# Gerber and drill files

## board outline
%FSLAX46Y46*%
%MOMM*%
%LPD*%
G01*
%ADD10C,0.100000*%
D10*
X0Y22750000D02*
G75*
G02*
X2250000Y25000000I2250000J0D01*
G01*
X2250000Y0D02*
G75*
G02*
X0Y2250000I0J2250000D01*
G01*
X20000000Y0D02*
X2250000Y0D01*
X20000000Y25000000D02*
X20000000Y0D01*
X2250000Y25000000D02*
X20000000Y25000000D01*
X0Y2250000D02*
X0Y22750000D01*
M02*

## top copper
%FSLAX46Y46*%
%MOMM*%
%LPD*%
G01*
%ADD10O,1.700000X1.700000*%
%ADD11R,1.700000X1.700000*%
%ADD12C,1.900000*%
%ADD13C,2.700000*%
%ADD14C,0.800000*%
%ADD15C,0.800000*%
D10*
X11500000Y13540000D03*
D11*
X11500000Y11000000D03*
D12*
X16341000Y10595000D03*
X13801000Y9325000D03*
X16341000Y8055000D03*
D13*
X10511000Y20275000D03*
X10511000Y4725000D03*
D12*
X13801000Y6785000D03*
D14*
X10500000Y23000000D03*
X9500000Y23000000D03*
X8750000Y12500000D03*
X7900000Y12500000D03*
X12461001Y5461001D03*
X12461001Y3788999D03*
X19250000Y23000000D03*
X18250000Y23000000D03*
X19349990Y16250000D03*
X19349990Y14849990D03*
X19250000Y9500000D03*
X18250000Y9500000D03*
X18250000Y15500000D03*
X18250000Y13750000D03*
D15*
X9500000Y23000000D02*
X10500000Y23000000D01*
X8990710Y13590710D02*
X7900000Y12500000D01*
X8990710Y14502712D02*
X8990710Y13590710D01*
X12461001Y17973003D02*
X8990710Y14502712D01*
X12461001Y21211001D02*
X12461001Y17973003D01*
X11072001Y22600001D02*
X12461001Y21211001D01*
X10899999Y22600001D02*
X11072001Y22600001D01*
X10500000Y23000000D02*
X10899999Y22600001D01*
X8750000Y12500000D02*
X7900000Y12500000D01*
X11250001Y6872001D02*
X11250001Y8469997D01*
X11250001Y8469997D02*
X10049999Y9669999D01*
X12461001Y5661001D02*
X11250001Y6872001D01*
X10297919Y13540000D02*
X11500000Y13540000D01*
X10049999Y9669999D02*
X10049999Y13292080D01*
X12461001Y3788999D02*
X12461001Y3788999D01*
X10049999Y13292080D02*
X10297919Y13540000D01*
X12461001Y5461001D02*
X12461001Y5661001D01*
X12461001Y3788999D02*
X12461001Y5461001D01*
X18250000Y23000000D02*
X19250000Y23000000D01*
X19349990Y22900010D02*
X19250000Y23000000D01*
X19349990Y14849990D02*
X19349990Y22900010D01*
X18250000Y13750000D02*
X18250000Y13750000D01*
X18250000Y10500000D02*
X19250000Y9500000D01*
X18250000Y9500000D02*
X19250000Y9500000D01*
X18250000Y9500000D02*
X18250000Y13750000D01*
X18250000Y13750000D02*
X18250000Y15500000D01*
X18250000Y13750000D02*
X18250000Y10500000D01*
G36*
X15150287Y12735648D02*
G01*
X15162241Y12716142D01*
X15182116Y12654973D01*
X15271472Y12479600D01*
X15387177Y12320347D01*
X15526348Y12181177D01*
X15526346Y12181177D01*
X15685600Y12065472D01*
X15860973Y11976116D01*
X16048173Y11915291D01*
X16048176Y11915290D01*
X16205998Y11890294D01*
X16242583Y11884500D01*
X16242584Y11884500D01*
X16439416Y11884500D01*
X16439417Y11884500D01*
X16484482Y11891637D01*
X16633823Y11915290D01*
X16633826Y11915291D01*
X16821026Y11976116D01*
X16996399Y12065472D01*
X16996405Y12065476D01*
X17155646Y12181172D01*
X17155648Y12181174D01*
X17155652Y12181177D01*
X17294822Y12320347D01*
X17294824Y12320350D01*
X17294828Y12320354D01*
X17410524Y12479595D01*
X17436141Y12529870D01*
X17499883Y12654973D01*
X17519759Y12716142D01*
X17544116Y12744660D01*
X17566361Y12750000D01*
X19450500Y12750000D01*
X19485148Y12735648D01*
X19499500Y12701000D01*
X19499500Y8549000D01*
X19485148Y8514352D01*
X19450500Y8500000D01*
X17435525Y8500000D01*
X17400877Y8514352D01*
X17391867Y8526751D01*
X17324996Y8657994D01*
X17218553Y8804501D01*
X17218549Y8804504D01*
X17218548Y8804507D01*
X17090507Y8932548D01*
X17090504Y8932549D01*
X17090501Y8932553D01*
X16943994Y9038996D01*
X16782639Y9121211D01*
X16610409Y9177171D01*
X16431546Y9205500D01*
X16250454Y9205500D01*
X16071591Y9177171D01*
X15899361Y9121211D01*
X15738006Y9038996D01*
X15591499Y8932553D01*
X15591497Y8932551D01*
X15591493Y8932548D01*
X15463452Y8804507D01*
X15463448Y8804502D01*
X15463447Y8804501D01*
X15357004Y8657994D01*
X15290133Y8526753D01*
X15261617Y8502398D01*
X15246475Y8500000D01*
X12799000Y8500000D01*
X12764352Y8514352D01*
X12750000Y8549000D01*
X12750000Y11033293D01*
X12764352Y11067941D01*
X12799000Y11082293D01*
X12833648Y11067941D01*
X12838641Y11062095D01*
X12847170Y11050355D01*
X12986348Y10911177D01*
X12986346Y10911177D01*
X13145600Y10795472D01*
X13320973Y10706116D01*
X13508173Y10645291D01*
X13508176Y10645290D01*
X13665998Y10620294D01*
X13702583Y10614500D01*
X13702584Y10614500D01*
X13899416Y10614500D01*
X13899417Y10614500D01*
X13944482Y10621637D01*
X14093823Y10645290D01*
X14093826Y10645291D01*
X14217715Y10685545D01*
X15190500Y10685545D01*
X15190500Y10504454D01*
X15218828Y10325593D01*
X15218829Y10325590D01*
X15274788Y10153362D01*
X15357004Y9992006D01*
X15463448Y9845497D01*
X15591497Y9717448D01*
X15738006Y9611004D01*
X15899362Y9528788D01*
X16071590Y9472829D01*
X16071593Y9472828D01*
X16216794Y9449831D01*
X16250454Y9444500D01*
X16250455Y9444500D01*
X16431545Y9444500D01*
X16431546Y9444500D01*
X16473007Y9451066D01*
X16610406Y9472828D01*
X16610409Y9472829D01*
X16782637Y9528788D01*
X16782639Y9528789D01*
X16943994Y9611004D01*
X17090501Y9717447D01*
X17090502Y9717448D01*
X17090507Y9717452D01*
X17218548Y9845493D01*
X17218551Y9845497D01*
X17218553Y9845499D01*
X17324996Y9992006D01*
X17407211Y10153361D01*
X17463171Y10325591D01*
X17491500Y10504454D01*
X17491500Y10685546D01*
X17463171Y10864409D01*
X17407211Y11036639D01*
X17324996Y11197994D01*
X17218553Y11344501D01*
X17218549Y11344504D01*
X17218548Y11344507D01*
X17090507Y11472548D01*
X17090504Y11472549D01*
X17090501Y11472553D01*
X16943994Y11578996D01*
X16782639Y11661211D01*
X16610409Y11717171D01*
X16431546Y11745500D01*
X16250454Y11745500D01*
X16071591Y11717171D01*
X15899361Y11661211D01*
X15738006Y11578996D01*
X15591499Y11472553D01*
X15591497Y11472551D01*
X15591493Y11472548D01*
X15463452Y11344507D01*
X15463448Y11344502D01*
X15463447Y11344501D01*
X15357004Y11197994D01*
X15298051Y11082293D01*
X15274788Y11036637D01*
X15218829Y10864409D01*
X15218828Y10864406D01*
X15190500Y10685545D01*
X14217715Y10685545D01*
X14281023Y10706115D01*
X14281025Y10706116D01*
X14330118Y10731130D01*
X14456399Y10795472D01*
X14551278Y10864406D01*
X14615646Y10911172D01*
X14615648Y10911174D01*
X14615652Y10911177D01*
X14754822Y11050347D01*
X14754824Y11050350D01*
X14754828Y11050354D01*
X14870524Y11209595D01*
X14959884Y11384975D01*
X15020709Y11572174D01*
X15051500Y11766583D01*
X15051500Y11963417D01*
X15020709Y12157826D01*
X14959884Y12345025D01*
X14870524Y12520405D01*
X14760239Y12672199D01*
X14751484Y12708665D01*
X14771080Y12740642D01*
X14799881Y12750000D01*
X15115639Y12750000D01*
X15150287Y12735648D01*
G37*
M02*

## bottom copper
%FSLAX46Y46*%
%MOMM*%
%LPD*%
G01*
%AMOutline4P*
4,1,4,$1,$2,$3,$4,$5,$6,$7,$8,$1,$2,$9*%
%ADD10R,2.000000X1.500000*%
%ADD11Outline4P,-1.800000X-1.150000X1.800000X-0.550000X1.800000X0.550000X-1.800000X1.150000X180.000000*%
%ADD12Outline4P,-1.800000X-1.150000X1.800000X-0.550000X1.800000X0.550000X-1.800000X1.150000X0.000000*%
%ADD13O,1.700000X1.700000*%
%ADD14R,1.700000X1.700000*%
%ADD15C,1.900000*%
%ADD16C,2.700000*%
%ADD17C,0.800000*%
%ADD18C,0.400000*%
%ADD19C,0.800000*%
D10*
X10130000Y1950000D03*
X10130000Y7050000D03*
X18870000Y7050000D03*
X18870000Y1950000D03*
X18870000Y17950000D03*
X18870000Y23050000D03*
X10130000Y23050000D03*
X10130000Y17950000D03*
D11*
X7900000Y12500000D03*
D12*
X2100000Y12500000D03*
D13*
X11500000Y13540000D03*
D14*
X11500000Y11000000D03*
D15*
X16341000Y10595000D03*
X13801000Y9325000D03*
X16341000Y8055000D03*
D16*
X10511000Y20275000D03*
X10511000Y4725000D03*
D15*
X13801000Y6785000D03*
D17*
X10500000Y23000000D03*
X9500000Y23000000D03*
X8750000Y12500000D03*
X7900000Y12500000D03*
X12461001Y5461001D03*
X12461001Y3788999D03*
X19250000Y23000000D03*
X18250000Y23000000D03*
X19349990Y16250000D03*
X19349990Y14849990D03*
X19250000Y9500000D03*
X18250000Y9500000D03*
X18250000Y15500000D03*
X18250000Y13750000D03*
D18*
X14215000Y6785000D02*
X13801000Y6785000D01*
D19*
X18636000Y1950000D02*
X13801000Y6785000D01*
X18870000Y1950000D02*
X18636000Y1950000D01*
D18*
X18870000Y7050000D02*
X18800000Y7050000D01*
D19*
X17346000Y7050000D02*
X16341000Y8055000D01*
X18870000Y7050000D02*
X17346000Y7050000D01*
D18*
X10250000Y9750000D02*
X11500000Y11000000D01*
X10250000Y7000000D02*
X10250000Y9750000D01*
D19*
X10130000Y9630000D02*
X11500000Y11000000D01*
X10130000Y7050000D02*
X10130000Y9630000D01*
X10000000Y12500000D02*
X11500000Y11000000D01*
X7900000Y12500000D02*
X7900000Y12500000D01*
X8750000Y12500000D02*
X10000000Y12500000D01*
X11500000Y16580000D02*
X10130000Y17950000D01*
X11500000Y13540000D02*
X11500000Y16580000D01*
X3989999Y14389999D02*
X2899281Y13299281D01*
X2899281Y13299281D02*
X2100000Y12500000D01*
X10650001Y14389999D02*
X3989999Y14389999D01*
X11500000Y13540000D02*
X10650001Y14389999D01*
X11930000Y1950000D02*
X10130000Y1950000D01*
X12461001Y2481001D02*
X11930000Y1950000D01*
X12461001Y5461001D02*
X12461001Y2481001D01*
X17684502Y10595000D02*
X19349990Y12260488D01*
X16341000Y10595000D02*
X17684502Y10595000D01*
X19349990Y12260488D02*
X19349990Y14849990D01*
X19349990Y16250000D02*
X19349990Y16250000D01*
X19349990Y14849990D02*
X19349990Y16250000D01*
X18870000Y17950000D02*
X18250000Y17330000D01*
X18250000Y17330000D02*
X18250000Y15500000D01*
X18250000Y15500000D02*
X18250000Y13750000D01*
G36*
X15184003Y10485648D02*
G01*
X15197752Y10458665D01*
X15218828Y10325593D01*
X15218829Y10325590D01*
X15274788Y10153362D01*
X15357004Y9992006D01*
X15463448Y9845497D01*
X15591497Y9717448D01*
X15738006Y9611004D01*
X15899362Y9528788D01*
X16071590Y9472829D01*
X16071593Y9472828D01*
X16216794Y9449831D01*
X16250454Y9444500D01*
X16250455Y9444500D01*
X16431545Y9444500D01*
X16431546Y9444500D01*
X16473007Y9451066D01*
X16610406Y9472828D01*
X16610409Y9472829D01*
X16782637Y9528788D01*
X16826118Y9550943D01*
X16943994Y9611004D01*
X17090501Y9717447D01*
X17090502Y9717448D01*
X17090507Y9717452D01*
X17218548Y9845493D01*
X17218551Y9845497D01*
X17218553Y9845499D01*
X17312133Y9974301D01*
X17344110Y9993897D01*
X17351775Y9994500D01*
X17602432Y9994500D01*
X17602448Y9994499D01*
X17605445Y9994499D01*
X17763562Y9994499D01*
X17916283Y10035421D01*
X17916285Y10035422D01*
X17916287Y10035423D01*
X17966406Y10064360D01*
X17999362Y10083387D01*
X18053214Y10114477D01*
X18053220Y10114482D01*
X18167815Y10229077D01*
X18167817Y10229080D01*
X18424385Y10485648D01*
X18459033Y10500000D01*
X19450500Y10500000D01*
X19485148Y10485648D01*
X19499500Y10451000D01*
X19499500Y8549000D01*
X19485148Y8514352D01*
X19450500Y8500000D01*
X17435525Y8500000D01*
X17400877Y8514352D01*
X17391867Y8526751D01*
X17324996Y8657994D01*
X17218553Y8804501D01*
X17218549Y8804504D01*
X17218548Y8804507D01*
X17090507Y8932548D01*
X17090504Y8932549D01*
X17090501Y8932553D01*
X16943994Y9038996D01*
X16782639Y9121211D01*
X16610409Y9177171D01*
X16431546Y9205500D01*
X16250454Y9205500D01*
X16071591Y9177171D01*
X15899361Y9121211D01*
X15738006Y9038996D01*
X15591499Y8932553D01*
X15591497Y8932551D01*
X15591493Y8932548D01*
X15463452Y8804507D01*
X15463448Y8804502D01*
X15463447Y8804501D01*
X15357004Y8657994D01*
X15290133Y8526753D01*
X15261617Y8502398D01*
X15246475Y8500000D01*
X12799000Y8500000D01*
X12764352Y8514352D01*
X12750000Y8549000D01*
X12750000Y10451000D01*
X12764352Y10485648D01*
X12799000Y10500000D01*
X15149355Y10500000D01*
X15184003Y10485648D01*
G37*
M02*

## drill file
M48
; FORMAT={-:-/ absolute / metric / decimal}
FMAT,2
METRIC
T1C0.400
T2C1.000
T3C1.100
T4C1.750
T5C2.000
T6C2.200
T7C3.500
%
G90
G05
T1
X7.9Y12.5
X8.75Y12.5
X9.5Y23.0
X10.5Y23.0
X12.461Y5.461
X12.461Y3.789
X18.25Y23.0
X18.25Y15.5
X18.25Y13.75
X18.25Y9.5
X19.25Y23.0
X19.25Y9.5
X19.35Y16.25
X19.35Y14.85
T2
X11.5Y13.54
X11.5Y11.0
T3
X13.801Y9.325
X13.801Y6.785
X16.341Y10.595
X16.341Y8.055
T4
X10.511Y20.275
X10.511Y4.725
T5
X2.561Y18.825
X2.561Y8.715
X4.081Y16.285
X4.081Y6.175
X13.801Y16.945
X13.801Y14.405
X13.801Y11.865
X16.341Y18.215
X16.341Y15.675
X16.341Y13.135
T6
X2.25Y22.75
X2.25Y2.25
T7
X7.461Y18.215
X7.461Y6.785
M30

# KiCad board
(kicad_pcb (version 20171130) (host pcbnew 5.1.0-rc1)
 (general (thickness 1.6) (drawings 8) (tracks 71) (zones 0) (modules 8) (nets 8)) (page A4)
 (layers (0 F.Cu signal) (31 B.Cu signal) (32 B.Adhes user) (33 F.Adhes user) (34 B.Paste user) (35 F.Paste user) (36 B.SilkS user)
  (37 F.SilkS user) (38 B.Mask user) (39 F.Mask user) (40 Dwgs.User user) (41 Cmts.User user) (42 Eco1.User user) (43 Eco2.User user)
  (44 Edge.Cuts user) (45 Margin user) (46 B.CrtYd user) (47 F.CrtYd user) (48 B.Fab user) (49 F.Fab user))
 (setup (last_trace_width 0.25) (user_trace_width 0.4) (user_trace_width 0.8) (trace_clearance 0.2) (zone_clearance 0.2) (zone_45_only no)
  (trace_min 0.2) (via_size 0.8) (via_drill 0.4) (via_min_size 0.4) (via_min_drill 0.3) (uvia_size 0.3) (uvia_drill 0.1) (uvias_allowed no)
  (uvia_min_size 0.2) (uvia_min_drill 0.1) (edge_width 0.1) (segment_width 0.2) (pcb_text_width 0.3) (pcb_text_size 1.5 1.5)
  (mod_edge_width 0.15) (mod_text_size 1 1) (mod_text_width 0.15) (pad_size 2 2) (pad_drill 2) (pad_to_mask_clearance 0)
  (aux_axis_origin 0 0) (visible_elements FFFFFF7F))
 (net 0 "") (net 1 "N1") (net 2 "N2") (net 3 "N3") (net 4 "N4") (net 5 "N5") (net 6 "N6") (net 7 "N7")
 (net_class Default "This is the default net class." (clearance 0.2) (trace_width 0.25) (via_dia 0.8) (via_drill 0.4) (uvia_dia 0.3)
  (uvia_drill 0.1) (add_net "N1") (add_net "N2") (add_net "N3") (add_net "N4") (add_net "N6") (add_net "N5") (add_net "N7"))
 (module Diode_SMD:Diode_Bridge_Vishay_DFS (layer B.Cu) (at 14.5 -4.5)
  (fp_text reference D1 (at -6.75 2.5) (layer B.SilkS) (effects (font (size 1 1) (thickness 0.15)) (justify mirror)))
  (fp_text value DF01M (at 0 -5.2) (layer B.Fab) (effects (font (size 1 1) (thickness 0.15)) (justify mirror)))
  (pad 1 smd rect (at -4.37 2.55) (size 2 1.5) (layers B.Cu B.Paste B.Mask) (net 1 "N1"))
  (pad 2 smd rect (at -4.37 -2.55) (size 2 1.5) (layers B.Cu B.Paste B.Mask) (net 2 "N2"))
  (pad 3 smd rect (at 4.37 -2.55) (size 2 1.5) (layers B.Cu B.Paste B.Mask) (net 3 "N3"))
  (pad 4 smd rect (at 4.37 2.55) (size 2 1.5) (layers B.Cu B.Paste B.Mask) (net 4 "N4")))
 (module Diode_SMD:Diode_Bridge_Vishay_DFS (layer B.Cu) (at 14.5 -20.5)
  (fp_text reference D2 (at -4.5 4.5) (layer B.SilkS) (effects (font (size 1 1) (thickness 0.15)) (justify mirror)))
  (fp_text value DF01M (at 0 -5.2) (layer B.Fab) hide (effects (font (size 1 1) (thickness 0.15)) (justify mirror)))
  (pad 4 smd rect (at 4.37 2.55) (size 2 1.5) (layers B.Cu B.Paste B.Mask) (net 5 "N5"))
  (pad 3 smd rect (at 4.37 -2.55) (size 2 1.5) (layers B.Cu B.Paste B.Mask) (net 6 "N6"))
  (pad 2 smd rect (at -4.37 -2.55) (size 2 1.5) (layers B.Cu B.Paste B.Mask) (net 2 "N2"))
  (pad 1 smd rect (at -4.37 2.55) (size 2 1.5) (layers B.Cu B.Paste B.Mask) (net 1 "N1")))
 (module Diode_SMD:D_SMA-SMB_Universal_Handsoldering (layer B.Cu) (at 5 -12.5)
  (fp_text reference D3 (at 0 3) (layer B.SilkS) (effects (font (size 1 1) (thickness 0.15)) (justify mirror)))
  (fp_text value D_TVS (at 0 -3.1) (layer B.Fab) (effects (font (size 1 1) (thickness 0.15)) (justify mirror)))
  (pad 2 smd trapezoid (at 2.9 0 180) (size 3.6 1.7) (rect_delta 0.6 0) (layers B.Cu B.Paste B.Mask) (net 2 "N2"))
  (pad 1 smd trapezoid (at -2.9 0) (size 3.6 1.7) (rect_delta 0.6 0) (layers B.Cu B.Paste B.Mask) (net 1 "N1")))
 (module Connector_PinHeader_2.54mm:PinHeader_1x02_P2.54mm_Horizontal (layer B.Cu) (at 11.5 -11)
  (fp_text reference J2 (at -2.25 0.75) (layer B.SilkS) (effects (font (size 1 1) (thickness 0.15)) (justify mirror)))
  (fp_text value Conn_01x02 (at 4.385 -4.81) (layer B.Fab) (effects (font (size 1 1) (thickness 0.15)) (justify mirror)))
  (pad 2 thru_hole oval (at 0 -2.54) (size 1.7 1.7) (drill 1) (layers *.Cu *.Mask) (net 1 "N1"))
  (pad 1 thru_hole rect (at 0 0) (size 1.7 1.7) (drill 1) (layers *.Cu *.Mask) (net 2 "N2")))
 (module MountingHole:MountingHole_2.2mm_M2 (layer F.Cu) (at 2.25 -2.25)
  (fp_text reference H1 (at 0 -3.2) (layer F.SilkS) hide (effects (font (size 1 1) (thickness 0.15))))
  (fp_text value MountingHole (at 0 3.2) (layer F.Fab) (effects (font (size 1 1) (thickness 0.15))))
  (pad 1 np_thru_hole circle (at 0 0) (size 2.2 2.2) (drill 2.2) (layers *.Cu *.Mask)))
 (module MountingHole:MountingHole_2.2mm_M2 (layer F.Cu) (at 2.25 -22.75)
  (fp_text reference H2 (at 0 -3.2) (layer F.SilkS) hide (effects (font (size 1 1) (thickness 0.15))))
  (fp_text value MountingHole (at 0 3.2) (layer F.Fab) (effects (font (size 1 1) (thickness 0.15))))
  (pad 1 np_thru_hole circle (at 0 0) (size 2.2 2.2) (drill 2.2) (layers *.Cu *.Mask)))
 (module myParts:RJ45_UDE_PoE (layer F.Cu) (at 16.341 -18.215 270)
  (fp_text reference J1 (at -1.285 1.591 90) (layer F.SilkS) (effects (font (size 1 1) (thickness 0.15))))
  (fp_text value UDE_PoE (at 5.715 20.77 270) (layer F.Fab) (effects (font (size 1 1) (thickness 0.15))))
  (pad "" np_thru_hole circle (at 2.54 0 270) (size 2 2) (drill 2) (layers *.Cu *.Mask))
  (pad "" np_thru_hole circle (at 3.81 2.54 270) (size 2 2) (drill 2) (layers *.Cu *.Mask))
  (pad "" np_thru_hole circle (at 5.08 0 270) (size 2 2) (drill 2) (layers *.Cu *.Mask))
  (pad "" np_thru_hole circle (at 6.35 2.54 270) (size 2 2) (drill 2) (layers *.Cu *.Mask))
  (pad R7 thru_hole circle (at 7.62 0 270) (size 1.9 1.9) (drill 1.1) (layers *.Cu *.Mask) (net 6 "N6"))
  (pad R8 thru_hole circle (at 8.89 2.54 270) (size 1.9 1.9) (drill 1.1) (layers *.Cu *.Mask) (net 5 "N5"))
  (pad R9 thru_hole circle (at 10.16 0 270) (size 1.9 1.9) (drill 1.1) (layers *.Cu *.Mask) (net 3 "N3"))
  (pad "" np_thru_hole circle (at 12.04 12.26 270) (size 2 2) (drill 2) (layers *.Cu *.Mask))
  (pad "" np_thru_hole circle (at 9.5 13.78 270) (size 2 2) (drill 2) (layers *.Cu *.Mask))
  (pad "" np_thru_hole circle (at 1.93 12.26 270) (size 2 2) (drill 2) (layers *.Cu *.Mask))
  (pad "" np_thru_hole circle (at -0.61 13.78 270) (size 2 2) (drill 2) (layers *.Cu *.Mask))
  (pad SH thru_hole circle (at -2.06 5.83 270) (size 2.7 2.7) (drill 1.75) (layers *.Cu *.Mask) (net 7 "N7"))
  (pad SH thru_hole circle (at 13.49 5.83 270) (size 2.7 2.7) (drill 1.75) (layers *.Cu *.Mask) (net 7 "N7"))
  (pad "" np_thru_hole circle (at 0 8.88 270) (size 3.5 3.5) (drill 3.5) (layers *.Cu *.Mask))
  (pad "" np_thru_hole circle (at 11.43 8.88 270) (size 3.5 3.5) (drill 3.5) (layers *.Cu *.Mask))
  (pad R10 thru_hole circle (at 11.43 2.54 270) (size 1.9 1.9) (drill 1.1) (layers *.Cu *.Mask) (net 4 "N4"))
  (pad "" np_thru_hole circle (at 0 0 270) (size 2 2) (drill 2) (layers *.Cu *.Mask))
  (pad "" np_thru_hole circle (at 1.27 2.54 270) (size 2 2) (drill 2) (layers *.Cu *.Mask)))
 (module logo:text (layer F.Cu) (at 18.5 -11 90)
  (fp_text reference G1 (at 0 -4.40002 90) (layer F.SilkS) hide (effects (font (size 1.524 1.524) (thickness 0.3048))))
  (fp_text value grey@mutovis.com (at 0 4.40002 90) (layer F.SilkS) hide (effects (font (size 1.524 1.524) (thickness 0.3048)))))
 (gr_arc (start 2.25 -22.75) (end 2.25 -25) (angle -90) (layer Edge.Cuts) (width 0.1))
 (gr_arc (start 2.25 -2.25) (end 0 -2.25) (angle -90) (layer Edge.Cuts) (width 0.1))
 (gr_line (start 20 0) (end 2.25 0) (layer Edge.Cuts) (width 0.1))
 (gr_line (start 20 -25) (end 20 0) (layer Edge.Cuts) (width 0.1))
 (gr_line (start 2.25 -25) (end 20 -25) (layer Edge.Cuts) (width 0.1))
 (gr_line (start 0 -2.25) (end 0 -22.75) (layer Edge.Cuts) (width 0.1))
 (segment (start 14.215 -6.785) (end 13.801 -6.785) (width 0.4) (layer B.Cu) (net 4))
 (segment (start 18.636 -1.95) (end 13.801 -6.785) (width 0.8) (layer B.Cu) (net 4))
 (segment (start 18.87 -1.95) (end 18.636 -1.95) (width 0.8) (layer B.Cu) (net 4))
 (segment (start 18.87 -7.05) (end 18.8 -7.05) (width 0.4) (layer B.Cu) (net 3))
 (segment (start 17.346 -7.05) (end 16.341 -8.055) (width 0.8) (layer B.Cu) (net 3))
 (segment (start 18.87 -7.05) (end 17.346 -7.05) (width 0.8) (layer B.Cu) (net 3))
 (via (at 10.5 -23) (size 0.8) (drill 0.4) (layers F.Cu B.Cu) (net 2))
 (via (at 9.5 -23) (size 0.8) (drill 0.4) (layers F.Cu B.Cu) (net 2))
 (segment (start 10.25 -9.75) (end 11.5 -11) (width 0.4) (layer B.Cu) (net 2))
 (segment (start 10.25 -7) (end 10.25 -9.75) (width 0.4) (layer B.Cu) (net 2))
 (segment (start 10.13 -9.63) (end 11.5 -11) (width 0.8) (layer B.Cu) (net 2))
 (segment (start 10.13 -7.05) (end 10.13 -9.63) (width 0.8) (layer B.Cu) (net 2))
 (segment (start 10 -12.5) (end 11.5 -11) (width 0.8) (layer B.Cu) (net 2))
 (segment (start 7.9 -12.5) (end 7.9 -12.5) (width 0.8) (layer B.Cu) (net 2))
 (segment (start 8.75 -12.5) (end 10 -12.5) (width 0.8) (layer B.Cu) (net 2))
 (via (at 8.75 -12.5) (size 0.8) (drill 0.4) (layers F.Cu B.Cu) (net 2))
 (via (at 7.9 -12.5) (size 0.8) (drill 0.4) (layers F.Cu B.Cu) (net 2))
 (segment (start 9.5 -23) (end 10.5 -23) (width 0.8) (layer F.Cu) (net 2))
 (segment (start 8.99071 -13.59071) (end 7.9 -12.5) (width 0.8) (layer F.Cu) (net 2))
 (segment (start 8.99071 -14.502712) (end 8.99071 -13.59071) (width 0.8) (layer F.Cu) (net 2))
 (segment (start 12.461001 -17.973003) (end 8.99071 -14.502712) (width 0.8) (layer F.Cu) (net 2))
 (segment (start 12.461001 -21.211001) (end 12.461001 -17.973003) (width 0.8) (layer F.Cu) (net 2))
 (segment (start 11.072001 -22.600001) (end 12.461001 -21.211001) (width 0.8) (layer F.Cu) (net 2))
 (segment (start 10.899999 -22.600001) (end 11.072001 -22.600001) (width 0.8) (layer F.Cu) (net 2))
 (segment (start 10.5 -23) (end 10.899999 -22.600001) (width 0.8) (layer F.Cu) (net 2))
 (segment (start 8.75 -12.5) (end 7.9 -12.5) (width 0.8) (layer F.Cu) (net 2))
 (segment (start 11.250001 -6.872001) (end 11.250001 -8.469997) (width 0.8) (layer F.Cu) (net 1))
 (segment (start 11.250001 -8.469997) (end 10.049999 -9.669999) (width 0.8) (layer F.Cu) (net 1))
 (segment (start 12.461001 -5.661001) (end 11.250001 -6.872001) (width 0.8) (layer F.Cu) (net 1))
 (segment (start 10.297919 -13.54) (end 11.5 -13.54) (width 0.8) (layer F.Cu) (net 1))
 (segment (start 10.049999 -9.669999) (end 10.049999 -13.29208) (width 0.8) (layer F.Cu) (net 1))
 (segment (start 12.461001 -3.788999) (end 12.461001 -3.788999) (width 0.8) (layer F.Cu) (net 1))
 (segment (start 10.049999 -13.29208) (end 10.297919 -13.54) (width 0.8) (layer F.Cu) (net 1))
 (segment (start 11.5 -16.58) (end 10.13 -17.95) (width 0.8) (layer B.Cu) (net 1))
 (segment (start 11.5 -13.54) (end 11.5 -16.58) (width 0.8) (layer B.Cu) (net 1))
 (segment (start 3.989999 -14.389999) (end 2.899281 -13.299281) (width 0.8) (layer B.Cu) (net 1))
 (segment (start 2.899281 -13.299281) (end 2.1 -12.5) (width 0.8) (layer B.Cu) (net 1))
 (segment (start 10.650001 -14.389999) (end 3.989999 -14.389999) (width 0.8) (layer B.Cu) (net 1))
 (segment (start 11.5 -13.54) (end 10.650001 -14.389999) (width 0.8) (layer B.Cu) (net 1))
 (segment (start 12.461001 -5.461001) (end 12.461001 -5.661001) (width 0.8) (layer F.Cu) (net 1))
 (via (at 12.461001 -5.461001) (size 0.8) (drill 0.4) (layers F.Cu B.Cu) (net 1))
 (segment (start 12.461001 -3.788999) (end 12.461001 -5.461001) (width 0.8) (layer F.Cu) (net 1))
 (via (at 12.461001 -3.788999) (size 0.8) (drill 0.4) (layers F.Cu B.Cu) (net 1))
 (segment (start 11.93 -1.95) (end 10.13 -1.95) (width 0.8) (layer B.Cu) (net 1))
 (segment (start 12.461001 -2.481001) (end 11.93 -1.95) (width 0.8) (layer B.Cu) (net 1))
 (segment (start 12.461001 -5.461001) (end 12.461001 -2.481001) (width 0.8) (layer B.Cu) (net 1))
 (via (at 19.25 -23) (size 0.8) (drill 0.4) (layers F.Cu B.Cu) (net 6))
 (via (at 18.25 -23) (size 0.8) (drill 0.4) (layers F.Cu B.Cu) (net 6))
 (segment (start 18.25 -23) (end 19.25 -23) (width 0.8) (layer F.Cu) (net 6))
 (segment (start 17.684502 -10.595) (end 19.34999 -12.260488) (width 0.8) (layer B.Cu) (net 6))
 (segment (start 16.341 -10.595) (end 17.684502 -10.595) (width 0.8) (layer B.Cu) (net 6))
 (segment (start 19.34999 -12.260488) (end 19.34999 -14.84999) (width 0.8) (layer B.Cu) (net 6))
 (segment (start 19.34999 -16.25) (end 19.34999 -16.25) (width 0.8) (layer B.Cu) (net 6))
 (via (at 19.34999 -16.25) (size 0.8) (drill 0.4) (layers F.Cu B.Cu) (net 6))
 (segment (start 19.34999 -14.84999) (end 19.34999 -16.25) (width 0.8) (layer B.Cu) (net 6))
 (via (at 19.34999 -14.84999) (size 0.8) (drill 0.4) (layers F.Cu B.Cu) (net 6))
 (segment (start 19.34999 -22.90001) (end 19.25 -23) (width 0.8) (layer F.Cu) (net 6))
 (segment (start 19.34999 -14.84999) (end 19.34999 -22.90001) (width 0.8) (layer F.Cu) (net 6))
 (segment (start 18.87 -17.95) (end 18.25 -17.33) (width 0.8) (layer B.Cu) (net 5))
 (segment (start 18.25 -17.33) (end 18.25 -15.5) (width 0.8) (layer B.Cu) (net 5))
 (via (at 19.25 -9.5) (size 0.8) (drill 0.4) (layers F.Cu B.Cu) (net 5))
 (segment (start 18.25 -13.75) (end 18.25 -13.75) (width 0.8) (layer F.Cu) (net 5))
 (segment (start 18.25 -10.5) (end 19.25 -9.5) (width 0.8) (layer F.Cu) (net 5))
 (via (at 18.25 -9.5) (size 0.8) (drill 0.4) (layers F.Cu B.Cu) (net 5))
 (segment (start 18.25 -9.5) (end 19.25 -9.5) (width 0.8) (layer F.Cu) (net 5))
 (segment (start 18.25 -9.5) (end 18.25 -13.75) (width 0.8) (layer F.Cu) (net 5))
 (segment (start 18.25 -15.5) (end 18.25 -13.75) (width 0.8) (layer B.Cu) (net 5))
 (via (at 18.25 -15.5) (size 0.8) (drill 0.4) (layers F.Cu B.Cu) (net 5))
 (segment (start 18.25 -13.75) (end 18.25 -15.5) (width 0.8) (layer F.Cu) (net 5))
 (segment (start 18.25 -13.75) (end 18.25 -10.5) (width 0.8) (layer F.Cu) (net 5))
 (via (at 18.25 -13.75) (size 0.8) (drill 0.4) (layers F.Cu B.Cu) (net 5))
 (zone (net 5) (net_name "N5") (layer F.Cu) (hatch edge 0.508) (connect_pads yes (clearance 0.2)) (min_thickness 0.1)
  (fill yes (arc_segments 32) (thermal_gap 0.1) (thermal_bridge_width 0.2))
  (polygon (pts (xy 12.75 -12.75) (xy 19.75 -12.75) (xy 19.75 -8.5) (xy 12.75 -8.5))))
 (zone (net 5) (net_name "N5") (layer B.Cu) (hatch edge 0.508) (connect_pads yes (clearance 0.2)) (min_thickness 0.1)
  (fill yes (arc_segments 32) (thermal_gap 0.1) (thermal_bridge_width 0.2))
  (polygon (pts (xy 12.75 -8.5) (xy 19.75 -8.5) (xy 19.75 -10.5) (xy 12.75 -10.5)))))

